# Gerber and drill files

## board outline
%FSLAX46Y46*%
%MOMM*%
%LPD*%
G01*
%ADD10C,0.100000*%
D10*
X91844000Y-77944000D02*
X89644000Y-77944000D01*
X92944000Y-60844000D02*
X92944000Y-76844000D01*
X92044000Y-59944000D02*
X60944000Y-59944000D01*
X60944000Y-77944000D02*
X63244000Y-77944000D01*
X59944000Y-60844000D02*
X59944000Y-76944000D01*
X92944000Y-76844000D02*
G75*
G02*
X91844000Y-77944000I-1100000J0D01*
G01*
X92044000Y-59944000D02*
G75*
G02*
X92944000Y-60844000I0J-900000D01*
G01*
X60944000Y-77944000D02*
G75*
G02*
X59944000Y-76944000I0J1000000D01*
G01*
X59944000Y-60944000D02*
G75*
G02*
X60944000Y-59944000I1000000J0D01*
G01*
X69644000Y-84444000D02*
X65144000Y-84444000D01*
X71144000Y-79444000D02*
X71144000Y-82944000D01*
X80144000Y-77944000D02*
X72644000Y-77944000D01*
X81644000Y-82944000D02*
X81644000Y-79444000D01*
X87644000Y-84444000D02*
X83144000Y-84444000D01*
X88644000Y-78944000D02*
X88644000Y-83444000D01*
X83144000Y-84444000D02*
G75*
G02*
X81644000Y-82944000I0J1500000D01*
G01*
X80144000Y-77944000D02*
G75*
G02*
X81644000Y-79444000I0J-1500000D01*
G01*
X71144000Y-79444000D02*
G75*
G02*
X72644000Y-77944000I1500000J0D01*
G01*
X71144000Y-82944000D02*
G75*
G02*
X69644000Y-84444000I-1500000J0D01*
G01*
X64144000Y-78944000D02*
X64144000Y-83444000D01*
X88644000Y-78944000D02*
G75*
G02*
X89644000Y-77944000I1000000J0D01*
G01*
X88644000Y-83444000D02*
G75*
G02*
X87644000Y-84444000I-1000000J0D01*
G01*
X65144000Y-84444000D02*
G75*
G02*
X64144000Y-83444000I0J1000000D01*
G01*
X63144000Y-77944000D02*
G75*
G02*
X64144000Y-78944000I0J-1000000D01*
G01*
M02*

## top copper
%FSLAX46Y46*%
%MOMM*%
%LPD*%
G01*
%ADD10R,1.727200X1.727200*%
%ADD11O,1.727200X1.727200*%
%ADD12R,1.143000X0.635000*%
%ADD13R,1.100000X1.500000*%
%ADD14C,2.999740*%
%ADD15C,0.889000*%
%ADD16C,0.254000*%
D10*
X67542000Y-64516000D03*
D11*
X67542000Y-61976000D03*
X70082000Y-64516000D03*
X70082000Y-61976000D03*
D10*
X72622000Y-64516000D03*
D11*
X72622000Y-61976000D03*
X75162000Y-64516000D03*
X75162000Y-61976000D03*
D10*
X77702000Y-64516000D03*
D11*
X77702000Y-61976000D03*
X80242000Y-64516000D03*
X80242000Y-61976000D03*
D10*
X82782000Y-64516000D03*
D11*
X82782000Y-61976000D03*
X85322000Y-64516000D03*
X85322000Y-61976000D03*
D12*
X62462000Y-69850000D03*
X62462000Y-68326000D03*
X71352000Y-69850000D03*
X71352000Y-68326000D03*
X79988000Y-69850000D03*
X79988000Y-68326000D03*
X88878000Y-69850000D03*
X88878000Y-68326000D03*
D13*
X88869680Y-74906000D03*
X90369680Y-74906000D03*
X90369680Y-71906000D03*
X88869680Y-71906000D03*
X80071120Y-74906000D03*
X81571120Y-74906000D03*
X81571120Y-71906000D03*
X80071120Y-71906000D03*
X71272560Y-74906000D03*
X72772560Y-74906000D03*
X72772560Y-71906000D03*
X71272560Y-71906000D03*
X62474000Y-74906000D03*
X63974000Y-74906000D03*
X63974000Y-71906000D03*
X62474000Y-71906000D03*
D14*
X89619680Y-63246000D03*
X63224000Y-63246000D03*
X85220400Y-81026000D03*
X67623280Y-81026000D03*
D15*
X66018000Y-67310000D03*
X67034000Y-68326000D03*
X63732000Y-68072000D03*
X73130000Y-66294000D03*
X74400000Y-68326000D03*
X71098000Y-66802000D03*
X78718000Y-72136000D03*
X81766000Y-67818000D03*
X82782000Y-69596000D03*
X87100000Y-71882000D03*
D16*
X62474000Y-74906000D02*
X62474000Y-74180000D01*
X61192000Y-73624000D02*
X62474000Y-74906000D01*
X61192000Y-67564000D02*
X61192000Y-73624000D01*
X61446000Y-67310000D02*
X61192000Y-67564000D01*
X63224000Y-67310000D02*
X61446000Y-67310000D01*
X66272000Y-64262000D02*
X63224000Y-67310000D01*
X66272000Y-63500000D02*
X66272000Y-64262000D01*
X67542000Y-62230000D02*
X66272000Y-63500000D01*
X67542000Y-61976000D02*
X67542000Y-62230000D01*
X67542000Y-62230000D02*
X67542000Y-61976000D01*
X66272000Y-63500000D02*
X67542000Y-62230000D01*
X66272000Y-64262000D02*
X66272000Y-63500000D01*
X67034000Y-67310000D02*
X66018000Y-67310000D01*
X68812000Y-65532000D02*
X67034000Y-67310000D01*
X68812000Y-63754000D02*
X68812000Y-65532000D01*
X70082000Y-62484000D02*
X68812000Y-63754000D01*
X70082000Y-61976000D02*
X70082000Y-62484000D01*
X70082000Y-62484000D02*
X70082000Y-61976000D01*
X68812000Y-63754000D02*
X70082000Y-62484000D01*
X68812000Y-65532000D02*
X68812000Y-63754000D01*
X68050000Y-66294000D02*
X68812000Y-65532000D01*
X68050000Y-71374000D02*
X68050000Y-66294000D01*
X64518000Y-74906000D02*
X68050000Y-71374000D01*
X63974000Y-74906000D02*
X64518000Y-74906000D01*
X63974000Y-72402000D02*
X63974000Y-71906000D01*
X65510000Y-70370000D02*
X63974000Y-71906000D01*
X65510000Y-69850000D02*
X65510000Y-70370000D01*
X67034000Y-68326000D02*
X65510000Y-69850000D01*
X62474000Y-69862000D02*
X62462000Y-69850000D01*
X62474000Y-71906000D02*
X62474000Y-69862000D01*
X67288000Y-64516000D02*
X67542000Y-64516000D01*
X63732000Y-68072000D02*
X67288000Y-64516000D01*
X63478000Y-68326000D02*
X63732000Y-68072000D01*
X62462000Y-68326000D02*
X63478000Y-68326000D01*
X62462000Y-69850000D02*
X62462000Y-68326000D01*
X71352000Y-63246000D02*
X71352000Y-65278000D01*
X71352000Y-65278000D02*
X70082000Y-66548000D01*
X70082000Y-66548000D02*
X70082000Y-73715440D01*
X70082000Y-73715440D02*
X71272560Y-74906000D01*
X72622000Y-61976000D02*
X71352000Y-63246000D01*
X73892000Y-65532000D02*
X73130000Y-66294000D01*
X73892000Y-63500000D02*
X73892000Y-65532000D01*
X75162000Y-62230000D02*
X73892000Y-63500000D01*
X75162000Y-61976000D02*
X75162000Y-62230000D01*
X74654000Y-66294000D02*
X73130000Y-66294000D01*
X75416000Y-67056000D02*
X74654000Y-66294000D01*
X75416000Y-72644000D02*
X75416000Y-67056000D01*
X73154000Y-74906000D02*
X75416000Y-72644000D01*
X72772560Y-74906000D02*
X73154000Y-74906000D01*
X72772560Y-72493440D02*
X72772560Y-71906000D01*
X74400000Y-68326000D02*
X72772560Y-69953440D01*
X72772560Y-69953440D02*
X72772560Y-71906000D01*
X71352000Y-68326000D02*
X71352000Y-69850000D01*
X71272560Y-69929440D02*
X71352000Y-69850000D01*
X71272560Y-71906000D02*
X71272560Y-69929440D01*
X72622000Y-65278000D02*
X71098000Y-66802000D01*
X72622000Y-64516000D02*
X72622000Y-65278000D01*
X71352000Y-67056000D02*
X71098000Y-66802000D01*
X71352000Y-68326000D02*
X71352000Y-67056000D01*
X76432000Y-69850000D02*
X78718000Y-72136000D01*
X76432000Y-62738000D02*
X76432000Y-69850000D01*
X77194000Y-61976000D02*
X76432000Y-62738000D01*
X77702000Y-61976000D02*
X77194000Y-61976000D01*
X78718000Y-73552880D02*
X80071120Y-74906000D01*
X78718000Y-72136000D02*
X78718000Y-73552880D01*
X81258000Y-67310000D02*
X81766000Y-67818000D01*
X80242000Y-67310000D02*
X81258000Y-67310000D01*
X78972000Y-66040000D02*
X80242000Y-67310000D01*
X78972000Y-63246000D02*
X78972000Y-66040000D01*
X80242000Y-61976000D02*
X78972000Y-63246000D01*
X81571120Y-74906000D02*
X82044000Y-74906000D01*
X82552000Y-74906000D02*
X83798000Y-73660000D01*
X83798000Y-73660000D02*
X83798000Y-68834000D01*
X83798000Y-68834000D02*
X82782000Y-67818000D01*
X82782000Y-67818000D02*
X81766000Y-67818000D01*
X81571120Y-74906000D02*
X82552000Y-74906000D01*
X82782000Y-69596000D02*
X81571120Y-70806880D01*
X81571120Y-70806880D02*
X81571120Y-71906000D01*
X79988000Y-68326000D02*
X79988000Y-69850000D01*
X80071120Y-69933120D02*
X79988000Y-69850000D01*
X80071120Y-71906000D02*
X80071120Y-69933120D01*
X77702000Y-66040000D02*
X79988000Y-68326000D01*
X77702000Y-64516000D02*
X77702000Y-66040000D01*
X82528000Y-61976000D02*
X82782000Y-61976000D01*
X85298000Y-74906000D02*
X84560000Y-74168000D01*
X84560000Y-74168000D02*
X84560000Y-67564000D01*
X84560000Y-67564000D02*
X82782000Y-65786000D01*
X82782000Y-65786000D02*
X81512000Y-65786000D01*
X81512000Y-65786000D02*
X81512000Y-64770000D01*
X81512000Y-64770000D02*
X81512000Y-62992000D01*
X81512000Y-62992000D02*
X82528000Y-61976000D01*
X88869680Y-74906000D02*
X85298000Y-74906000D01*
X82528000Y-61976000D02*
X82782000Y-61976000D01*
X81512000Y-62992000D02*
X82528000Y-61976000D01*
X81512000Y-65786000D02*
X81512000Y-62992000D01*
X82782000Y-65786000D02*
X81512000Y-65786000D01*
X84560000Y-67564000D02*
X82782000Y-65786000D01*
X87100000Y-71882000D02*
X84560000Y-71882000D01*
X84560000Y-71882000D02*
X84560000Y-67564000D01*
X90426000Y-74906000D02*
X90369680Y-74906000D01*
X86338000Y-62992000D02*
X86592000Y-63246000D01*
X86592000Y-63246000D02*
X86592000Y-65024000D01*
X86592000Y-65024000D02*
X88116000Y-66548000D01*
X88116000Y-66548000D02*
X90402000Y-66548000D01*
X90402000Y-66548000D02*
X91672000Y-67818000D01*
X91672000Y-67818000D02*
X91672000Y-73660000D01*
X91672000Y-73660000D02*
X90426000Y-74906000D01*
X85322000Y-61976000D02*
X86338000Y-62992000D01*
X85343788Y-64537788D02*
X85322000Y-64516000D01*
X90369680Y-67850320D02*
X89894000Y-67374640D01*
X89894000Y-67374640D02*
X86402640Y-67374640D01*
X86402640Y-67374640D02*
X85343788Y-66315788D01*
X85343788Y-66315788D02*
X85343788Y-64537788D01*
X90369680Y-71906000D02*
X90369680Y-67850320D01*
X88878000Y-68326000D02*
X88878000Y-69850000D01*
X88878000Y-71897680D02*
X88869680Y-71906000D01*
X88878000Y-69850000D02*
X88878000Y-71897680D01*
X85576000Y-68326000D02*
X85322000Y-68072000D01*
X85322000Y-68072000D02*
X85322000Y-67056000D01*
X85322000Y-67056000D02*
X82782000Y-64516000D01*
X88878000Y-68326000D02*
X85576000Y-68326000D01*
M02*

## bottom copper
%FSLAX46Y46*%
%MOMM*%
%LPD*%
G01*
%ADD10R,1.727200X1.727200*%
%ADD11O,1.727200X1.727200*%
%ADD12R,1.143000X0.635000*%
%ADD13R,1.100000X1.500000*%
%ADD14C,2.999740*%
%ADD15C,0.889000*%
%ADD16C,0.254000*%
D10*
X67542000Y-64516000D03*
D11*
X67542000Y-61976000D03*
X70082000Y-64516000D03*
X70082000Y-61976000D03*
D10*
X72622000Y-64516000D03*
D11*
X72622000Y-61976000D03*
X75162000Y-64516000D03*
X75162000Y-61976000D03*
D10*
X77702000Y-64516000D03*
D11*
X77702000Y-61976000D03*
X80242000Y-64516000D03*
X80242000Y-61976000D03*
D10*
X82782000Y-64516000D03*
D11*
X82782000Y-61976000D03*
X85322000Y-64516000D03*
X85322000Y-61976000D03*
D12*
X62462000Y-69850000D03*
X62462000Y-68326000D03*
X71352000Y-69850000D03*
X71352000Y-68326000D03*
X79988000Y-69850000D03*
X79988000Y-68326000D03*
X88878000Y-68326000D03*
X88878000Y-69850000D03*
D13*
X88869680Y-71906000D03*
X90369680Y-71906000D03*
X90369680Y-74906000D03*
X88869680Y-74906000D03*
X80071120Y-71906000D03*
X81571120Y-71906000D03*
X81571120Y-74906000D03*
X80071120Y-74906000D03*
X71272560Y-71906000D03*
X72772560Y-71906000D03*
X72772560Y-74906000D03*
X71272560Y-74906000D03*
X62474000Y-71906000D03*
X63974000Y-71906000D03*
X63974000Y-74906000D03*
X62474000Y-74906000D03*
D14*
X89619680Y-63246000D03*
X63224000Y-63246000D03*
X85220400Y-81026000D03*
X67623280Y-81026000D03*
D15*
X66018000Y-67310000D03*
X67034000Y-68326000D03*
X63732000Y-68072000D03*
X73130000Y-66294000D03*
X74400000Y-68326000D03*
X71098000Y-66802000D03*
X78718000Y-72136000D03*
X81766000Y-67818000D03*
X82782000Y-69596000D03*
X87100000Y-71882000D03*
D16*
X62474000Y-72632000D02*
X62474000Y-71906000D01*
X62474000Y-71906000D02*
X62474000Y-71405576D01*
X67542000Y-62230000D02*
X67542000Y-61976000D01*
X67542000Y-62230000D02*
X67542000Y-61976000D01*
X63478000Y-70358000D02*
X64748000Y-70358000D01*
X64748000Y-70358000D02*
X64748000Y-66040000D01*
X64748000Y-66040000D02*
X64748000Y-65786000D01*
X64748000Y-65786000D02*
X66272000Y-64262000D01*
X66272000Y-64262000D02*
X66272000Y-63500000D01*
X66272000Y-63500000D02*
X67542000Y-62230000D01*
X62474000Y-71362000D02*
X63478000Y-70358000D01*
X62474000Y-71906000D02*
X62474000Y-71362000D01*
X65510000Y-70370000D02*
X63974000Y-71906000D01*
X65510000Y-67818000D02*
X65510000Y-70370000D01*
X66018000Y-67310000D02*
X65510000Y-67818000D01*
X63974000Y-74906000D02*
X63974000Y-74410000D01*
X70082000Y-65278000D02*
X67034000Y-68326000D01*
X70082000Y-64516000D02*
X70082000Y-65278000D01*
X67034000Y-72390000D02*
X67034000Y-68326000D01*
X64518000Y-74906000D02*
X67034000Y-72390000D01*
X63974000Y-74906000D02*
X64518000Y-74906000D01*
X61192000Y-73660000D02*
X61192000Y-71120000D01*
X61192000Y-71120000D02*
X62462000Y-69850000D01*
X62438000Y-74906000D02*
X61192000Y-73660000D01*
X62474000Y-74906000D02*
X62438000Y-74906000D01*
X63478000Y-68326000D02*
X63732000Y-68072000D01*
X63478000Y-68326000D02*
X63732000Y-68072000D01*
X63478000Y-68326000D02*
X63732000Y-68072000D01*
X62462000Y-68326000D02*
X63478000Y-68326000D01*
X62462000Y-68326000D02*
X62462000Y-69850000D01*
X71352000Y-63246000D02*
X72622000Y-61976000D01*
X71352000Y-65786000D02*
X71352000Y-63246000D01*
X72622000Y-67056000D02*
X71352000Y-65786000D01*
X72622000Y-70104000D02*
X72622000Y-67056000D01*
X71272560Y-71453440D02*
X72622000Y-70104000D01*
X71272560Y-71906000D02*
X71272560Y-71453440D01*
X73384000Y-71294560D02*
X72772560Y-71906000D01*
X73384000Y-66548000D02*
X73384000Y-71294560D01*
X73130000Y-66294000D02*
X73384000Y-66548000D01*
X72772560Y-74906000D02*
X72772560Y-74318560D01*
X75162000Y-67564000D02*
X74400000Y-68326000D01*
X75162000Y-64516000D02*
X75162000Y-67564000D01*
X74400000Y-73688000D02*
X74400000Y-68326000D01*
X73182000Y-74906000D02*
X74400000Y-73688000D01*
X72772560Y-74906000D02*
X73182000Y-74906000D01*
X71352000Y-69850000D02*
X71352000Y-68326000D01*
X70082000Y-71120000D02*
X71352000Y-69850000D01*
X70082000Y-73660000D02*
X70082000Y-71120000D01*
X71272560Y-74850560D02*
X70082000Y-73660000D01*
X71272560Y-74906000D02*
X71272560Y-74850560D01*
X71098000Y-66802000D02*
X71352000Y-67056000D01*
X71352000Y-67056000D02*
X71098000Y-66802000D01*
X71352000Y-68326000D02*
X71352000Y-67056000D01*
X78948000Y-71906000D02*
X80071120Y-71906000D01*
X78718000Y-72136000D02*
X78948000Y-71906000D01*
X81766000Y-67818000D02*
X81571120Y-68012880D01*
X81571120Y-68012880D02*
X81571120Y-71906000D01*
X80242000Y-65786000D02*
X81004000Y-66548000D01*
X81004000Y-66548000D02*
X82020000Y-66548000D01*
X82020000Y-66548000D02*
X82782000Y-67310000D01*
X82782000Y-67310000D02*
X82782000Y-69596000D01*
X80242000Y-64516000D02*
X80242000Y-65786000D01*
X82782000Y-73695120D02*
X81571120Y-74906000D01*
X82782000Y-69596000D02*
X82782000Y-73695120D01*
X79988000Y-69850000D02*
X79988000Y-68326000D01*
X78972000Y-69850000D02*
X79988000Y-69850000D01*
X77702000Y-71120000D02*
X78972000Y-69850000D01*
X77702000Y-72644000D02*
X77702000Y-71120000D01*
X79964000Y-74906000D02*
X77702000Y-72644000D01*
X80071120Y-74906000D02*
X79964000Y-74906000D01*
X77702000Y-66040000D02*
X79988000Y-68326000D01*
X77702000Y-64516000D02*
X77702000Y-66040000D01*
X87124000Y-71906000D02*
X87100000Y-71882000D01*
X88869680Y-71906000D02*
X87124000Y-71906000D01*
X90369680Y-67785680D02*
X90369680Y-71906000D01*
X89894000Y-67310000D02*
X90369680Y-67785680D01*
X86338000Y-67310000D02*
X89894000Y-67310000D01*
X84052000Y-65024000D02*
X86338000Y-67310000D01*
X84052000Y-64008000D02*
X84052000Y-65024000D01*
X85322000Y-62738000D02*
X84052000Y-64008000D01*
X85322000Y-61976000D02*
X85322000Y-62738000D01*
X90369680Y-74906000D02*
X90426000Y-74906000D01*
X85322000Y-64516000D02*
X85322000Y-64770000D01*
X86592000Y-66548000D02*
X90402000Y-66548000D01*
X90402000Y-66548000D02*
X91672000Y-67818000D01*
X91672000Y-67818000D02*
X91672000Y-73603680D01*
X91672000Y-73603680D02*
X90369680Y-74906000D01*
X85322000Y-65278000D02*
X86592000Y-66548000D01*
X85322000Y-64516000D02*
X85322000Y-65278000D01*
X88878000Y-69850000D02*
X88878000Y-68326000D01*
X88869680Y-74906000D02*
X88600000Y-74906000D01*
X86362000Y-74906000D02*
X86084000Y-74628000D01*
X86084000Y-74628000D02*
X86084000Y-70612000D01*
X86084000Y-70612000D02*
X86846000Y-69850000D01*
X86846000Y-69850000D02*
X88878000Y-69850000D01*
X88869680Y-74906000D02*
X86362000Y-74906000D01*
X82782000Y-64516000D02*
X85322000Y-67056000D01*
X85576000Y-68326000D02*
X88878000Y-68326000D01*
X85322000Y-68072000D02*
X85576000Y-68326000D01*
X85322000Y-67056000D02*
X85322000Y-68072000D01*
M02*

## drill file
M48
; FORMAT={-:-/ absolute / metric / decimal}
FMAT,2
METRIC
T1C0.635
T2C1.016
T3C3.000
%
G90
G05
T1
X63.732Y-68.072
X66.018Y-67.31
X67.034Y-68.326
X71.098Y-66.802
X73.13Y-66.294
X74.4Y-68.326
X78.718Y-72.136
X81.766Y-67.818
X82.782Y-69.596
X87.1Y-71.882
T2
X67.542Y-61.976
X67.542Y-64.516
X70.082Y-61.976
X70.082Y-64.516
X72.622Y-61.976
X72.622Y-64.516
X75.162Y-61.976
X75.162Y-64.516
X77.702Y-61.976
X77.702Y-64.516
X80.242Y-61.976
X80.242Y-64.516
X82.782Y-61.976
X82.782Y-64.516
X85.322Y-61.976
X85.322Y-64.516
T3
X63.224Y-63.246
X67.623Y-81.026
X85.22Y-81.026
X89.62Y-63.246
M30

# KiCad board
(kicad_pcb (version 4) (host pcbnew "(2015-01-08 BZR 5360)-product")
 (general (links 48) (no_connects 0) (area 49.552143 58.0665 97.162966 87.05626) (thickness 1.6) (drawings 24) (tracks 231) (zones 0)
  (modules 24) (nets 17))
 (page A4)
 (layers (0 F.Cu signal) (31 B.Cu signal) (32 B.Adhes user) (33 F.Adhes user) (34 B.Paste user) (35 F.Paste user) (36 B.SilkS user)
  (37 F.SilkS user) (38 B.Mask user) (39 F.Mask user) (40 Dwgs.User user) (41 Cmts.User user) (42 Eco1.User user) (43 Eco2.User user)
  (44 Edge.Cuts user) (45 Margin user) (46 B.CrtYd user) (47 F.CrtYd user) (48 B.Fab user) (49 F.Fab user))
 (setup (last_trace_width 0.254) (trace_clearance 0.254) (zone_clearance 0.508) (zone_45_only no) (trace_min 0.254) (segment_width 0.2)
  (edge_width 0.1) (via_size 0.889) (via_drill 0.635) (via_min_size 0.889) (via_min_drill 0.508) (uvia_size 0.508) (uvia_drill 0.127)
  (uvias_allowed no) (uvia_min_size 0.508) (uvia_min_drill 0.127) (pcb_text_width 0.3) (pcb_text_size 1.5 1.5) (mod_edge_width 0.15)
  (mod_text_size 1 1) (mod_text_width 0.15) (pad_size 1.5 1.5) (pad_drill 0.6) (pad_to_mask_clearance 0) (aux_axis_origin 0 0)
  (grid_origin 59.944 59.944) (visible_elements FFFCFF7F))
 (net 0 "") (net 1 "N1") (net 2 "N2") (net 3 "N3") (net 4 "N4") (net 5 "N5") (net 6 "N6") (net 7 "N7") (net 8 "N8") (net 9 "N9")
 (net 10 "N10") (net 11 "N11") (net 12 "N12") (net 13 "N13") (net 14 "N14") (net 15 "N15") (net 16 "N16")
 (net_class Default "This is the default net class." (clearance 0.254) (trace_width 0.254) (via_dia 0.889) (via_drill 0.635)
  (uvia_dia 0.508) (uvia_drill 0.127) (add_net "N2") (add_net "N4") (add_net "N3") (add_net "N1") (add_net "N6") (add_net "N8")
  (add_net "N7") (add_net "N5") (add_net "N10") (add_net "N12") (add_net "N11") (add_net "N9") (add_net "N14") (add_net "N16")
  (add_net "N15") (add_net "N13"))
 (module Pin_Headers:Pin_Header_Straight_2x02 (layer F.Cu) (at 68.812 63.246)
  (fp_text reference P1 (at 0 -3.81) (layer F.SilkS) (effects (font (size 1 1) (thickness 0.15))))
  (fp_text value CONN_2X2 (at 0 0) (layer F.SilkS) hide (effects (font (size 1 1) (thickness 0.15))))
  (pad 1 thru_hole rect (at -1.27 1.27) (size 1.7272 1.7272) (drill 1.016) (layers *.Cu *.Mask F.SilkS) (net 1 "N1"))
  (pad 2 thru_hole oval (at -1.27 -1.27) (size 1.7272 1.7272) (drill 1.016) (layers *.Cu *.Mask F.SilkS) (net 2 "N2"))
  (pad 3 thru_hole oval (at 1.27 1.27) (size 1.7272 1.7272) (drill 1.016) (layers *.Cu *.Mask F.SilkS) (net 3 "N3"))
  (pad 4 thru_hole oval (at 1.27 -1.27) (size 1.7272 1.7272) (drill 1.016) (layers *.Cu *.Mask F.SilkS) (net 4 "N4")))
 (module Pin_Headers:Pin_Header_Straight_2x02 (layer F.Cu) (at 73.892 63.246)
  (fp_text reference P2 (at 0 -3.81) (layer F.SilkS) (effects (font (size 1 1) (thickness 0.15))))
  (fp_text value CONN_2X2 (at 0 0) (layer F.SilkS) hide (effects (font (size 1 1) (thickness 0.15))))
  (pad 1 thru_hole rect (at -1.27 1.27) (size 1.7272 1.7272) (drill 1.016) (layers *.Cu *.Mask F.SilkS) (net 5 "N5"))
  (pad 2 thru_hole oval (at -1.27 -1.27) (size 1.7272 1.7272) (drill 1.016) (layers *.Cu *.Mask F.SilkS) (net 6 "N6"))
  (pad 3 thru_hole oval (at 1.27 1.27) (size 1.7272 1.7272) (drill 1.016) (layers *.Cu *.Mask F.SilkS) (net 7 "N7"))
  (pad 4 thru_hole oval (at 1.27 -1.27) (size 1.7272 1.7272) (drill 1.016) (layers *.Cu *.Mask F.SilkS) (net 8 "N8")))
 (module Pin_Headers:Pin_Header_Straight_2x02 (layer F.Cu) (at 78.972 63.246)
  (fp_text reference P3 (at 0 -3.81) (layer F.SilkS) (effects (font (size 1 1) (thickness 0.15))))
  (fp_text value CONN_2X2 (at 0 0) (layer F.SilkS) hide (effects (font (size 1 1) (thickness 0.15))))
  (pad 1 thru_hole rect (at -1.27 1.27) (size 1.7272 1.7272) (drill 1.016) (layers *.Cu *.Mask F.SilkS) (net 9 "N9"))
  (pad 2 thru_hole oval (at -1.27 -1.27) (size 1.7272 1.7272) (drill 1.016) (layers *.Cu *.Mask F.SilkS) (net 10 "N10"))
  (pad 3 thru_hole oval (at 1.27 1.27) (size 1.7272 1.7272) (drill 1.016) (layers *.Cu *.Mask F.SilkS) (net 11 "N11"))
  (pad 4 thru_hole oval (at 1.27 -1.27) (size 1.7272 1.7272) (drill 1.016) (layers *.Cu *.Mask F.SilkS) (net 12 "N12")))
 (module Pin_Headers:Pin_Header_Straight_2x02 (layer F.Cu) (at 84.052 63.246)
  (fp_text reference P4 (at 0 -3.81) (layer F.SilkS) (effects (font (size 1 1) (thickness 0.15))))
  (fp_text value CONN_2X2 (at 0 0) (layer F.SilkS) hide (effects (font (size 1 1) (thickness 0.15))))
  (pad 1 thru_hole rect (at -1.27 1.27) (size 1.7272 1.7272) (drill 1.016) (layers *.Cu *.Mask F.SilkS) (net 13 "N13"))
  (pad 2 thru_hole oval (at -1.27 -1.27) (size 1.7272 1.7272) (drill 1.016) (layers *.Cu *.Mask F.SilkS) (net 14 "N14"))
  (pad 3 thru_hole oval (at 1.27 1.27) (size 1.7272 1.7272) (drill 1.016) (layers *.Cu *.Mask F.SilkS) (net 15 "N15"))
  (pad 4 thru_hole oval (at 1.27 -1.27) (size 1.7272 1.7272) (drill 1.016) (layers *.Cu *.Mask F.SilkS) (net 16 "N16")))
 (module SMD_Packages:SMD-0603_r (layer F.Cu) (at 62.462 69.088 90)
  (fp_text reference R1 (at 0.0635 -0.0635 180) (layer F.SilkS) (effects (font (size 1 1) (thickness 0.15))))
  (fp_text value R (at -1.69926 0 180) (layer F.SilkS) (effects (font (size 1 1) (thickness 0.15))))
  (pad 1 smd rect (at -0.762 0 90) (size 0.635 1.143) (layers F.Cu F.Paste F.Mask) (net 1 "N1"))
  (pad 2 smd rect (at 0.762 0 90) (size 0.635 1.143) (layers F.Cu F.Paste F.Mask) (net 1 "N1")))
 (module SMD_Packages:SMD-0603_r (layer B.Cu) (at 62.462 69.088 90)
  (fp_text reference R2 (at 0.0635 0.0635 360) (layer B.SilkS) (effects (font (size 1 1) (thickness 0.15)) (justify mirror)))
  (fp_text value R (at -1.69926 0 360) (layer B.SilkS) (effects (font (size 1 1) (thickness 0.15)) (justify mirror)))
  (pad 1 smd rect (at -0.762 0 90) (size 0.635 1.143) (layers B.Cu B.Paste B.Mask) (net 1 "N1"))
  (pad 2 smd rect (at 0.762 0 90) (size 0.635 1.143) (layers B.Cu B.Paste B.Mask) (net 1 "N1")))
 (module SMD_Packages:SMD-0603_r (layer F.Cu) (at 71.352 69.088 90)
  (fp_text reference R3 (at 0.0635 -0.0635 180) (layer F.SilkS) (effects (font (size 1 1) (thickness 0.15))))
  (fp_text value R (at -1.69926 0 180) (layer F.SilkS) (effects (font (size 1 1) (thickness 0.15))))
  (pad 1 smd rect (at -0.762 0 90) (size 0.635 1.143) (layers F.Cu F.Paste F.Mask) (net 5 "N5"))
  (pad 2 smd rect (at 0.762 0 90) (size 0.635 1.143) (layers F.Cu F.Paste F.Mask) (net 5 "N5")))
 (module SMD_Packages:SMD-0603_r (layer B.Cu) (at 71.352 69.088 90)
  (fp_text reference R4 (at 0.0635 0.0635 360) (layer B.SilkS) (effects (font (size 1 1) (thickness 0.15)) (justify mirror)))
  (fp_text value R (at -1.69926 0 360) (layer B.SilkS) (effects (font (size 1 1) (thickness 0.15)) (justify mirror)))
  (pad 1 smd rect (at -0.762 0 90) (size 0.635 1.143) (layers B.Cu B.Paste B.Mask) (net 5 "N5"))
  (pad 2 smd rect (at 0.762 0 90) (size 0.635 1.143) (layers B.Cu B.Paste B.Mask) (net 5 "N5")))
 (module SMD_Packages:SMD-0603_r (layer F.Cu) (at 79.988 69.088 90)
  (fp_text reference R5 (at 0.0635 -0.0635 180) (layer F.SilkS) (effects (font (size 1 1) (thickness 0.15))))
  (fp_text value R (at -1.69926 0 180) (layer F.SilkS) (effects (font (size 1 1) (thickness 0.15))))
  (pad 1 smd rect (at -0.762 0 90) (size 0.635 1.143) (layers F.Cu F.Paste F.Mask) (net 9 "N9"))
  (pad 2 smd rect (at 0.762 0 90) (size 0.635 1.143) (layers F.Cu F.Paste F.Mask) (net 9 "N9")))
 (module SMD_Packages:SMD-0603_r (layer B.Cu) (at 79.988 69.088 90)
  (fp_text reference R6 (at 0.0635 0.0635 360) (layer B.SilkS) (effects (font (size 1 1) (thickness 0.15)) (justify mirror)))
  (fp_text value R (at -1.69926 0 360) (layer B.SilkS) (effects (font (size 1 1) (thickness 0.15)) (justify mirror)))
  (pad 1 smd rect (at -0.762 0 90) (size 0.635 1.143) (layers B.Cu B.Paste B.Mask) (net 9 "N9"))
  (pad 2 smd rect (at 0.762 0 90) (size 0.635 1.143) (layers B.Cu B.Paste B.Mask) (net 9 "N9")))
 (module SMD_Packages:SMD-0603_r (layer F.Cu) (at 88.878 69.088 90)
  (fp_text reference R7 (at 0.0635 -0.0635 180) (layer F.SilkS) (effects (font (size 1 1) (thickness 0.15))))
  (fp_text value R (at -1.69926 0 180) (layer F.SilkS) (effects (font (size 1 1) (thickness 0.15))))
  (pad 1 smd rect (at -0.762 0 90) (size 0.635 1.143) (layers F.Cu F.Paste F.Mask) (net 13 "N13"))
  (pad 2 smd rect (at 0.762 0 90) (size 0.635 1.143) (layers F.Cu F.Paste F.Mask) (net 13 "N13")))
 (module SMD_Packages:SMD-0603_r (layer B.Cu) (at 88.878 69.088 270)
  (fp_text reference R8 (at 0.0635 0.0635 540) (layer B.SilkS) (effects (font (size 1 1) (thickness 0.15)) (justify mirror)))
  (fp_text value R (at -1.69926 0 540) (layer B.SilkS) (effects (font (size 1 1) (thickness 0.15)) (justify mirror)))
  (pad 1 smd rect (at -0.762 0 270) (size 0.635 1.143) (layers B.Cu B.Paste B.Mask) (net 13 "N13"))
  (pad 2 smd rect (at 0.762 0 270) (size 0.635 1.143) (layers B.Cu B.Paste B.Mask) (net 13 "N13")))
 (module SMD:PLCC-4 (layer B.Cu) (at 89.61968 73.406 270)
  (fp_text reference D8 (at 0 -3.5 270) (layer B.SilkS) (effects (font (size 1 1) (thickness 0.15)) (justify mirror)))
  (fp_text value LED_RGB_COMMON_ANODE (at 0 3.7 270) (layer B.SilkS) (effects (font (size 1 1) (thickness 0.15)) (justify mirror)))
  (pad 1 smd rect (at -1.5 0.75) (size 1.1 1.5) (layers B.Cu B.Paste B.Mask) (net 14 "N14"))
  (pad 2 smd rect (at -1.5 -0.75) (size 1.1 1.5) (layers B.Cu B.Paste B.Mask) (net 16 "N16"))
  (pad 3 smd rect (at 1.5 -0.75) (size 1.1 1.5) (layers B.Cu B.Paste B.Mask) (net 15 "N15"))
  (pad 4 smd rect (at 1.5 0.75) (size 1.1 1.5) (layers B.Cu B.Paste B.Mask) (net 13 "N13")))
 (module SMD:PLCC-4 (layer F.Cu) (at 89.61968 73.406 90)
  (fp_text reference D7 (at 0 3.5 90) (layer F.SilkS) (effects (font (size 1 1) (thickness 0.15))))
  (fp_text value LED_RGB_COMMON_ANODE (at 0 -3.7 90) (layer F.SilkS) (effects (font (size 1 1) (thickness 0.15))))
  (pad 1 smd rect (at -1.5 -0.75) (size 1.1 1.5) (layers F.Cu F.Paste F.Mask) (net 14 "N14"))
  (pad 2 smd rect (at -1.5 0.75) (size 1.1 1.5) (layers F.Cu F.Paste F.Mask) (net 16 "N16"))
  (pad 3 smd rect (at 1.5 0.75) (size 1.1 1.5) (layers F.Cu F.Paste F.Mask) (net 15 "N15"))
  (pad 4 smd rect (at 1.5 -0.75) (size 1.1 1.5) (layers F.Cu F.Paste F.Mask) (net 13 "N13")))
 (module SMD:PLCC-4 (layer B.Cu) (at 80.82112 73.406 270)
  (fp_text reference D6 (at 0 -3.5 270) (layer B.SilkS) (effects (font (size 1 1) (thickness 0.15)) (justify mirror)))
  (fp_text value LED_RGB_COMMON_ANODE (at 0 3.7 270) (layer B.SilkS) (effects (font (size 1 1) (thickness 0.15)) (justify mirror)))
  (pad 1 smd rect (at -1.5 0.75) (size 1.1 1.5) (layers B.Cu B.Paste B.Mask) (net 10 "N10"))
  (pad 2 smd rect (at -1.5 -0.75) (size 1.1 1.5) (layers B.Cu B.Paste B.Mask) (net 12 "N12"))
  (pad 3 smd rect (at 1.5 -0.75) (size 1.1 1.5) (layers B.Cu B.Paste B.Mask) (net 11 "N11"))
  (pad 4 smd rect (at 1.5 0.75) (size 1.1 1.5) (layers B.Cu B.Paste B.Mask) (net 9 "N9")))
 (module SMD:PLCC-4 (layer F.Cu) (at 80.82112 73.406 90)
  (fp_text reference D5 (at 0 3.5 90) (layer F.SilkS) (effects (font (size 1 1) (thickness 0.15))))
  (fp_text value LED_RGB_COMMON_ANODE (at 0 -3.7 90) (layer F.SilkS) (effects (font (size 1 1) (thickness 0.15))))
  (pad 1 smd rect (at -1.5 -0.75) (size 1.1 1.5) (layers F.Cu F.Paste F.Mask) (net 10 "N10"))
  (pad 2 smd rect (at -1.5 0.75) (size 1.1 1.5) (layers F.Cu F.Paste F.Mask) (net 12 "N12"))
  (pad 3 smd rect (at 1.5 0.75) (size 1.1 1.5) (layers F.Cu F.Paste F.Mask) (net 11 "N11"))
  (pad 4 smd rect (at 1.5 -0.75) (size 1.1 1.5) (layers F.Cu F.Paste F.Mask) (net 9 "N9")))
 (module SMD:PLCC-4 (layer B.Cu) (at 72.02256 73.406 270)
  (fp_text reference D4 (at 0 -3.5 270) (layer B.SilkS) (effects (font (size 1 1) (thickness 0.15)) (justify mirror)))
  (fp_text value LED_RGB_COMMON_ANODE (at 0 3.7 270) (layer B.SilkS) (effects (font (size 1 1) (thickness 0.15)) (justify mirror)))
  (pad 1 smd rect (at -1.5 0.75) (size 1.1 1.5) (layers B.Cu B.Paste B.Mask) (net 6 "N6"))
  (pad 2 smd rect (at -1.5 -0.75) (size 1.1 1.5) (layers B.Cu B.Paste B.Mask) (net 8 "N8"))
  (pad 3 smd rect (at 1.5 -0.75) (size 1.1 1.5) (layers B.Cu B.Paste B.Mask) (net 7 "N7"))
  (pad 4 smd rect (at 1.5 0.75) (size 1.1 1.5) (layers B.Cu B.Paste B.Mask) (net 5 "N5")))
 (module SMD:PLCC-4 (layer F.Cu) (at 72.02256 73.406 90)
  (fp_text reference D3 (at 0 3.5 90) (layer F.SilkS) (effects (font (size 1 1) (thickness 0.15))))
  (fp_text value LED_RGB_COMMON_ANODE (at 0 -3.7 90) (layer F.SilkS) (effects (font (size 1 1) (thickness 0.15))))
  (pad 1 smd rect (at -1.5 -0.75) (size 1.1 1.5) (layers F.Cu F.Paste F.Mask) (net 6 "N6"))
  (pad 2 smd rect (at -1.5 0.75) (size 1.1 1.5) (layers F.Cu F.Paste F.Mask) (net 8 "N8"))
  (pad 3 smd rect (at 1.5 0.75) (size 1.1 1.5) (layers F.Cu F.Paste F.Mask) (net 7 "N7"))
  (pad 4 smd rect (at 1.5 -0.75) (size 1.1 1.5) (layers F.Cu F.Paste F.Mask) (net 5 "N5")))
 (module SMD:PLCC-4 (layer B.Cu) (at 63.224 73.406 270)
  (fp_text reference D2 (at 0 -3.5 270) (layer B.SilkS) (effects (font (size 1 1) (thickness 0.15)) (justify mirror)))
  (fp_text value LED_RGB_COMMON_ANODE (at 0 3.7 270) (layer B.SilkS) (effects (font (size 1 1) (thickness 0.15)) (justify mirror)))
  (pad 1 smd rect (at -1.5 0.75) (size 1.1 1.5) (layers B.Cu B.Paste B.Mask) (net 2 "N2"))
  (pad 2 smd rect (at -1.5 -0.75) (size 1.1 1.5) (layers B.Cu B.Paste B.Mask) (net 4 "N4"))
  (pad 3 smd rect (at 1.5 -0.75) (size 1.1 1.5) (layers B.Cu B.Paste B.Mask) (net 3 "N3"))
  (pad 4 smd rect (at 1.5 0.75) (size 1.1 1.5) (layers B.Cu B.Paste B.Mask) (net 1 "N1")))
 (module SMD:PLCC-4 (layer F.Cu) (at 63.224 73.406 90)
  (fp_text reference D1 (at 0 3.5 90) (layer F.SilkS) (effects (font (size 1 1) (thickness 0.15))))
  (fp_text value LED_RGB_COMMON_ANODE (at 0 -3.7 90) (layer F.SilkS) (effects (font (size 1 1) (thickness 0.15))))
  (pad 1 smd rect (at -1.5 -0.75) (size 1.1 1.5) (layers F.Cu F.Paste F.Mask) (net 2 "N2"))
  (pad 2 smd rect (at -1.5 0.75) (size 1.1 1.5) (layers F.Cu F.Paste F.Mask) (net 4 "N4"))
  (pad 3 smd rect (at 1.5 0.75) (size 1.1 1.5) (layers F.Cu F.Paste F.Mask) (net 3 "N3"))
  (pad 4 smd rect (at 1.5 -0.75) (size 1.1 1.5) (layers F.Cu F.Paste F.Mask) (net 1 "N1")))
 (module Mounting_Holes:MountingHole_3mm (layer F.Cu) (at 89.61968 63.246)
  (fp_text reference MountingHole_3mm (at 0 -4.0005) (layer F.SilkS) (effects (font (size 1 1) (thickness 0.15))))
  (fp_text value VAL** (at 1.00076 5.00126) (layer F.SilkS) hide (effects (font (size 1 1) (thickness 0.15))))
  (pad 1 thru_hole circle (at 0 0) (size 2.99974 2.99974) (drill 2.99974) (layers)))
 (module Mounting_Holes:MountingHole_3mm (layer F.Cu) (at 63.224 63.246)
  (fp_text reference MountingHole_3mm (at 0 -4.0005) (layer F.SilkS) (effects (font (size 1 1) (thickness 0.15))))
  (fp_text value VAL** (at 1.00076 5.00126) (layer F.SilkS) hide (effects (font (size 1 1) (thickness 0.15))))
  (pad 1 thru_hole circle (at 0 0) (size 2.99974 2.99974) (drill 2.99974) (layers)))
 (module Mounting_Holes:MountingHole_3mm (layer F.Cu) (at 85.2204 81.026)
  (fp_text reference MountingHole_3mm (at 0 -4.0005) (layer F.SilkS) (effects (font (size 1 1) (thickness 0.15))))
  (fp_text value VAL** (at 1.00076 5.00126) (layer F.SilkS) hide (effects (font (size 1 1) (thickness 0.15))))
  (pad 1 thru_hole circle (at 0 0) (size 2.99974 2.99974) (drill 2.99974) (layers)))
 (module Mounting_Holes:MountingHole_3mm (layer F.Cu) (at 67.62328 81.026)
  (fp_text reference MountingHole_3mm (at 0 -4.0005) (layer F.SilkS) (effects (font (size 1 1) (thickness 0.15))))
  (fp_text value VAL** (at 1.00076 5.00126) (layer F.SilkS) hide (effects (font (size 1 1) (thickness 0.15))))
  (pad 1 thru_hole circle (at 0 0) (size 2.99974 2.99974) (drill 2.99974) (layers)))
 (gr_line (start 91.844 77.944) (end 89.644 77.944) (angle 90) (layer Edge.Cuts) (width 0.1))
 (gr_line (start 92.944 60.844) (end 92.944 76.844) (angle 90) (layer Edge.Cuts) (width 0.1))
 (gr_line (start 92.044 59.944) (end 60.944 59.944) (angle 90) (layer Edge.Cuts) (width 0.1))
 (gr_line (start 60.944 77.944) (end 63.244 77.944) (angle 90) (layer Edge.Cuts) (width 0.1))
 (gr_line (start 59.944 60.844) (end 59.944 76.944) (angle 90) (layer Edge.Cuts) (width 0.1))
 (gr_arc (start 91.844 76.844) (end 92.944 76.844) (angle 90) (layer Edge.Cuts) (width 0.1))
 (gr_arc (start 92.044 60.844) (end 92.044 59.944) (angle 90) (layer Edge.Cuts) (width 0.1))
 (gr_arc (start 60.944 76.944) (end 60.944 77.944) (angle 90) (layer Edge.Cuts) (width 0.1))
 (gr_arc (start 60.944 60.944) (end 59.944 60.944) (angle 90) (layer Edge.Cuts) (width 0.1))
 (gr_line (start 69.644 84.444) (end 65.144 84.444) (angle 90) (layer Edge.Cuts) (width 0.1))
 (gr_line (start 71.144 79.444) (end 71.144 82.944) (angle 90) (layer Edge.Cuts) (width 0.1))
 (gr_line (start 80.144 77.944) (end 72.644 77.944) (angle 90) (layer Edge.Cuts) (width 0.1))
 (gr_line (start 81.644 82.944) (end 81.644 79.444) (angle 90) (layer Edge.Cuts) (width 0.1))
 (gr_line (start 87.644 84.444) (end 83.144 84.444) (angle 90) (layer Edge.Cuts) (width 0.1))
 (gr_line (start 88.644 78.944) (end 88.644 83.444) (angle 90) (layer Edge.Cuts) (width 0.1))
 (gr_arc (start 83.144 82.944) (end 83.144 84.444) (angle 90) (layer Edge.Cuts) (width 0.1))
 (gr_arc (start 80.144 79.444) (end 80.144 77.944) (angle 90) (layer Edge.Cuts) (width 0.1))
 (gr_arc (start 72.644 79.444) (end 71.144 79.444) (angle 90) (layer Edge.Cuts) (width 0.1))
 (gr_arc (start 69.644 82.944) (end 71.144 82.944) (angle 90) (layer Edge.Cuts) (width 0.1))
 (gr_line (start 64.144 78.944) (end 64.144 83.444) (angle 90) (layer Edge.Cuts) (width 0.1))
 (gr_arc (start 89.644 78.944) (end 88.644 78.944) (angle 90) (layer Edge.Cuts) (width 0.1))
 (gr_arc (start 87.644 83.444) (end 88.644 83.444) (angle 90) (layer Edge.Cuts) (width 0.1))
 (gr_arc (start 65.144 83.444) (end 65.144 84.444) (angle 90) (layer Edge.Cuts) (width 0.1))
 (gr_arc (start 63.144 78.944) (end 63.144 77.944) (angle 90) (layer Edge.Cuts) (width 0.1))
 (segment (start 62.474 72.632) (end 62.474 71.906) (width 0.254) (layer B.Cu) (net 2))
 (segment (start 62.474 74.906) (end 62.474 74.18) (width 0.254) (layer F.Cu) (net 2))
 (segment (start 62.474 71.906) (end 62.474 71.405576) (width 0.254) (layer B.Cu) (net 2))
 (segment (start 61.192 73.624) (end 62.474 74.906) (width 0.254) (layer F.Cu) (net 2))
 (segment (start 61.192 67.564) (end 61.192 73.624) (width 0.254) (layer F.Cu) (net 2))
 (segment (start 61.446 67.31) (end 61.192 67.564) (width 0.254) (layer F.Cu) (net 2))
 (segment (start 63.224 67.31) (end 61.446 67.31) (width 0.254) (layer F.Cu) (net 2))
 (segment (start 66.272 64.262) (end 63.224 67.31) (width 0.254) (layer F.Cu) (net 2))
 (segment (start 66.272 63.5) (end 66.272 64.262) (width 0.254) (layer F.Cu) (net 2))
 (segment (start 67.542 62.23) (end 66.272 63.5) (width 0.254) (layer F.Cu) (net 2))
 (segment (start 67.542 61.976) (end 67.542 62.23) (width 0.254) (layer F.Cu) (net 2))
 (segment (start 67.542 62.23) (end 67.542 61.976) (width 0.254) (layer F.Cu) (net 2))
 (segment (start 66.272 63.5) (end 67.542 62.23) (width 0.254) (layer F.Cu) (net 2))
 (segment (start 66.272 64.262) (end 66.272 63.5) (width 0.254) (layer F.Cu) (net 2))
 (segment (start 67.542 62.23) (end 67.542 61.976) (width 0.254) (layer B.Cu) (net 2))
 (segment (start 67.542 62.23) (end 67.542 61.976) (width 0.254) (layer B.Cu) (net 2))
 (segment (start 63.478 70.358) (end 64.748 70.358) (width 0.254) (layer B.Cu) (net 2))
 (segment (start 64.748 70.358) (end 64.748 66.04) (width 0.254) (layer B.Cu) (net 2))
 (segment (start 64.748 66.04) (end 64.748 65.786) (width 0.254) (layer B.Cu) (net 2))
 (segment (start 64.748 65.786) (end 66.272 64.262) (width 0.254) (layer B.Cu) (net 2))
 (segment (start 66.272 64.262) (end 66.272 63.5) (width 0.254) (layer B.Cu) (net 2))
 (segment (start 66.272 63.5) (end 67.542 62.23) (width 0.254) (layer B.Cu) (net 2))
 (segment (start 62.474 71.362) (end 63.478 70.358) (width 0.254) (layer B.Cu) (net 2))
 (segment (start 62.474 71.906) (end 62.474 71.362) (width 0.254) (layer B.Cu) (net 2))
 (segment (start 65.51 70.37) (end 63.974 71.906) (width 0.254) (layer B.Cu) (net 4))
 (segment (start 65.51 67.818) (end 65.51 70.37) (width 0.254) (layer B.Cu) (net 4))
 (segment (start 66.018 67.31) (end 65.51 67.818) (width 0.254) (layer B.Cu) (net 4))
 (via (at 66.018 67.31) (size 0.889) (layers F.Cu B.Cu) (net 4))
 (segment (start 67.034 67.31) (end 66.018 67.31) (width 0.254) (layer F.Cu) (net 4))
 (segment (start 68.812 65.532) (end 67.034 67.31) (width 0.254) (layer F.Cu) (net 4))
 (segment (start 68.812 63.754) (end 68.812 65.532) (width 0.254) (layer F.Cu) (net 4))
 (segment (start 70.082 62.484) (end 68.812 63.754) (width 0.254) (layer F.Cu) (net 4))
 (segment (start 70.082 61.976) (end 70.082 62.484) (width 0.254) (layer F.Cu) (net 4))
 (segment (start 70.082 62.484) (end 70.082 61.976) (width 0.254) (layer F.Cu) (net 4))
 (segment (start 68.812 63.754) (end 70.082 62.484) (width 0.254) (layer F.Cu) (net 4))
 (segment (start 68.812 65.532) (end 68.812 63.754) (width 0.254) (layer F.Cu) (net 4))
 (segment (start 68.05 66.294) (end 68.812 65.532) (width 0.254) (layer F.Cu) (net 4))
 (segment (start 68.05 71.374) (end 68.05 66.294) (width 0.254) (layer F.Cu) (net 4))
 (segment (start 64.518 74.906) (end 68.05 71.374) (width 0.254) (layer F.Cu) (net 4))
 (segment (start 63.974 74.906) (end 64.518 74.906) (width 0.254) (layer F.Cu) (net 4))
 (segment (start 63.974 72.402) (end 63.974 71.906) (width 0.254) (layer F.Cu) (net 3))
 (segment (start 63.974 74.906) (end 63.974 74.41) (width 0.254) (layer B.Cu) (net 3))
 (segment (start 65.51 70.37) (end 63.974 71.906) (width 0.254) (layer F.Cu) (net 3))
 (segment (start 65.51 69.85) (end 65.51 70.37) (width 0.254) (layer F.Cu) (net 3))
 (segment (start 67.034 68.326) (end 65.51 69.85) (width 0.254) (layer F.Cu) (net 3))
 (via (at 67.034 68.326) (size 0.889) (layers F.Cu B.Cu) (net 3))
 (segment (start 70.082 65.278) (end 67.034 68.326) (width 0.254) (layer B.Cu) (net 3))
 (segment (start 70.082 64.516) (end 70.082 65.278) (width 0.254) (layer B.Cu) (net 3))
 (segment (start 67.034 72.39) (end 67.034 68.326) (width 0.254) (layer B.Cu) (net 3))
 (segment (start 64.518 74.906) (end 67.034 72.39) (width 0.254) (layer B.Cu) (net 3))
 (segment (start 63.974 74.906) (end 64.518 74.906) (width 0.254) (layer B.Cu) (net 3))
 (segment (start 62.474 69.862) (end 62.462 69.85) (width 0.254) (layer F.Cu) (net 1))
 (segment (start 62.474 71.906) (end 62.474 69.862) (width 0.254) (layer F.Cu) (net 1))
 (segment (start 61.192 73.66) (end 61.192 71.12) (width 0.254) (layer B.Cu) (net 1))
 (segment (start 61.192 71.12) (end 62.462 69.85) (width 0.254) (layer B.Cu) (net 1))
 (segment (start 62.438 74.906) (end 61.192 73.66) (width 0.254) (layer B.Cu) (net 1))
 (segment (start 62.474 74.906) (end 62.438 74.906) (width 0.254) (layer B.Cu) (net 1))
 (segment (start 67.288 64.516) (end 67.542 64.516) (width 0.254) (layer F.Cu) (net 1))
 (segment (start 63.478 68.326) (end 63.732 68.072) (width 0.254) (layer B.Cu) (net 1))
 (via (at 63.732 68.072) (size 0.889) (layers F.Cu B.Cu) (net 1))
 (segment (start 63.732 68.072) (end 67.288 64.516) (width 0.254) (layer F.Cu) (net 1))
 (segment (start 63.478 68.326) (end 63.732 68.072) (width 0.254) (layer B.Cu) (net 1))
 (segment (start 63.478 68.326) (end 63.732 68.072) (width 0.254) (layer F.Cu) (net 1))
 (segment (start 62.462 68.326) (end 63.478 68.326) (width 0.254) (layer F.Cu) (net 1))
 (segment (start 63.478 68.326) (end 63.732 68.072) (width 0.254) (layer B.Cu) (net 1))
 (segment (start 62.462 68.326) (end 63.478 68.326) (width 0.254) (layer B.Cu) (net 1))
 (segment (start 62.462 68.326) (end 62.462 69.85) (width 0.254) (layer B.Cu) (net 1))
 (segment (start 62.462 69.85) (end 62.462 68.326) (width 0.254) (layer F.Cu) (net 1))
 (segment (start 71.352 63.246) (end 71.352 65.278) (width 0.254) (layer F.Cu) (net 6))
 (segment (start 71.352 65.278) (end 70.082 66.548) (width 0.254) (layer F.Cu) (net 6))
 (segment (start 70.082 66.548) (end 70.082 73.71544) (width 0.254) (layer F.Cu) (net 6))
 (segment (start 70.082 73.71544) (end 71.27256 74.906) (width 0.254) (layer F.Cu) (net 6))
 (segment (start 72.622 61.976) (end 71.352 63.246) (width 0.254) (layer F.Cu) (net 6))
 (segment (start 71.352 63.246) (end 72.622 61.976) (width 0.254) (layer B.Cu) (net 6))
 (segment (start 71.352 65.786) (end 71.352 63.246) (width 0.254) (layer B.Cu) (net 6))
 (segment (start 72.622 67.056) (end 71.352 65.786) (width 0.254) (layer B.Cu) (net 6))
 (segment (start 72.622 70.104) (end 72.622 67.056) (width 0.254) (layer B.Cu) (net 6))
 (segment (start 71.27256 71.45344) (end 72.622 70.104) (width 0.254) (layer B.Cu) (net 6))
 (segment (start 71.27256 71.906) (end 71.27256 71.45344) (width 0.254) (layer B.Cu) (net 6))
 (segment (start 73.384 71.29456) (end 72.77256 71.906) (width 0.254) (layer B.Cu) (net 8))
 (segment (start 73.384 66.548) (end 73.384 71.29456) (width 0.254) (layer B.Cu) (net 8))
 (segment (start 73.13 66.294) (end 73.384 66.548) (width 0.254) (layer B.Cu) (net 8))
 (via (at 73.13 66.294) (size 0.889) (layers F.Cu B.Cu) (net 8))
 (segment (start 73.892 65.532) (end 73.13 66.294) (width 0.254) (layer F.Cu) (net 8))
 (segment (start 73.892 63.5) (end 73.892 65.532) (width 0.254) (layer F.Cu) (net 8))
 (segment (start 75.162 62.23) (end 73.892 63.5) (width 0.254) (layer F.Cu) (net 8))
 (segment (start 75.162 61.976) (end 75.162 62.23) (width 0.254) (layer F.Cu) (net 8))
 (segment (start 74.654 66.294) (end 73.13 66.294) (width 0.254) (layer F.Cu) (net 8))
 (segment (start 75.416 67.056) (end 74.654 66.294) (width 0.254) (layer F.Cu) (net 8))
 (segment (start 75.416 72.644) (end 75.416 67.056) (width 0.254) (layer F.Cu) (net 8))
 (segment (start 73.154 74.906) (end 75.416 72.644) (width 0.254) (layer F.Cu) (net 8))
 (segment (start 72.77256 74.906) (end 73.154 74.906) (width 0.254) (layer F.Cu) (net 8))
 (segment (start 72.77256 72.49344) (end 72.77256 71.906) (width 0.254) (layer F.Cu) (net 7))
 (segment (start 72.77256 74.906) (end 72.77256 74.31856) (width 0.254) (layer B.Cu) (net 7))
 (segment (start 75.162 67.564) (end 74.4 68.326) (width 0.254) (layer B.Cu) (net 7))
 (via (at 74.4 68.326) (size 0.889) (layers F.Cu B.Cu) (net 7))
 (segment (start 74.4 68.326) (end 72.77256 69.95344) (width 0.254) (layer F.Cu) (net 7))
 (segment (start 72.77256 69.95344) (end 72.77256 71.906) (width 0.254) (layer F.Cu) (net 7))
 (segment (start 75.162 64.516) (end 75.162 67.564) (width 0.254) (layer B.Cu) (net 7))
 (segment (start 74.4 73.688) (end 74.4 68.326) (width 0.254) (layer B.Cu) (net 7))
 (segment (start 73.182 74.906) (end 74.4 73.688) (width 0.254) (layer B.Cu) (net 7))
 (segment (start 72.77256 74.906) (end 73.182 74.906) (width 0.254) (layer B.Cu) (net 7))
 (segment (start 71.352 69.85) (end 71.352 68.326) (width 0.254) (layer B.Cu) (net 5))
 (segment (start 71.352 68.326) (end 71.352 69.85) (width 0.254) (layer F.Cu) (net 5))
 (segment (start 71.27256 69.92944) (end 71.352 69.85) (width 0.254) (layer F.Cu) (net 5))
 (segment (start 71.27256 71.906) (end 71.27256 69.92944) (width 0.254) (layer F.Cu) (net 5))
 (segment (start 70.082 71.12) (end 71.352 69.85) (width 0.254) (layer B.Cu) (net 5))
 (segment (start 70.082 73.66) (end 70.082 71.12) (width 0.254) (layer B.Cu) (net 5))
 (segment (start 71.27256 74.85056) (end 70.082 73.66) (width 0.254) (layer B.Cu) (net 5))
 (segment (start 71.27256 74.906) (end 71.27256 74.85056) (width 0.254) (layer B.Cu) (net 5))
 (segment (start 71.098 66.802) (end 71.352 67.056) (width 0.254) (layer B.Cu) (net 5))
 (via (at 71.098 66.802) (size 0.889) (layers F.Cu B.Cu) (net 5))
 (segment (start 72.622 65.278) (end 71.098 66.802) (width 0.254) (layer F.Cu) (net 5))
 (segment (start 72.622 64.516) (end 72.622 65.278) (width 0.254) (layer F.Cu) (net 5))
 (segment (start 71.352 67.056) (end 71.098 66.802) (width 0.254) (layer F.Cu) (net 5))
 (segment (start 71.352 68.326) (end 71.352 67.056) (width 0.254) (layer F.Cu) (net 5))
 (segment (start 71.352 67.056) (end 71.098 66.802) (width 0.254) (layer B.Cu) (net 5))
 (segment (start 71.352 68.326) (end 71.352 67.056) (width 0.254) (layer B.Cu) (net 5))
 (segment (start 78.948 71.906) (end 80.07112 71.906) (width 0.254) (layer B.Cu) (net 10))
 (segment (start 78.718 72.136) (end 78.948 71.906) (width 0.254) (layer B.Cu) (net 10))
 (via (at 78.718 72.136) (size 0.889) (layers F.Cu B.Cu) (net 10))
 (segment (start 76.432 69.85) (end 78.718 72.136) (width 0.254) (layer F.Cu) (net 10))
 (segment (start 76.432 62.738) (end 76.432 69.85) (width 0.254) (layer F.Cu) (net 10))
 (segment (start 77.194 61.976) (end 76.432 62.738) (width 0.254) (layer F.Cu) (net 10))
 (segment (start 77.702 61.976) (end 77.194 61.976) (width 0.254) (layer F.Cu) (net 10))
 (segment (start 78.718 73.55288) (end 80.07112 74.906) (width 0.254) (layer F.Cu) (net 10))
 (segment (start 78.718 72.136) (end 78.718 73.55288) (width 0.254) (layer F.Cu) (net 10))
 (segment (start 81.766 67.818) (end 81.57112 68.01288) (width 0.254) (layer B.Cu) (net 12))
 (via (at 81.766 67.818) (size 0.889) (layers F.Cu B.Cu) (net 12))
 (segment (start 81.57112 68.01288) (end 81.57112 71.906) (width 0.254) (layer B.Cu) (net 12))
 (segment (start 81.258 67.31) (end 81.766 67.818) (width 0.254) (layer F.Cu) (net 12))
 (segment (start 80.242 67.31) (end 81.258 67.31) (width 0.254) (layer F.Cu) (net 12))
 (segment (start 78.972 66.04) (end 80.242 67.31) (width 0.254) (layer F.Cu) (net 12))
 (segment (start 78.972 63.246) (end 78.972 66.04) (width 0.254) (layer F.Cu) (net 12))
 (segment (start 80.242 61.976) (end 78.972 63.246) (width 0.254) (layer F.Cu) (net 12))
 (segment (start 81.57112 74.906) (end 82.044 74.906) (width 0.254) (layer F.Cu) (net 12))
 (segment (start 82.552 74.906) (end 83.798 73.66) (width 0.254) (layer F.Cu) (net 12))
 (segment (start 83.798 73.66) (end 83.798 68.834) (width 0.254) (layer F.Cu) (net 12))
 (segment (start 83.798 68.834) (end 82.782 67.818) (width 0.254) (layer F.Cu) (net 12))
 (segment (start 82.782 67.818) (end 81.766 67.818) (width 0.254) (layer F.Cu) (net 12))
 (segment (start 81.57112 74.906) (end 82.552 74.906) (width 0.254) (layer F.Cu) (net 12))
 (segment (start 80.242 65.786) (end 81.004 66.548) (width 0.254) (layer B.Cu) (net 11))
 (segment (start 81.004 66.548) (end 82.02 66.548) (width 0.254) (layer B.Cu) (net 11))
 (segment (start 82.02 66.548) (end 82.782 67.31) (width 0.254) (layer B.Cu) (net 11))
 (segment (start 82.782 67.31) (end 82.782 69.596) (width 0.254) (layer B.Cu) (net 11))
 (via (at 82.782 69.596) (size 0.889) (layers F.Cu B.Cu) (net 11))
 (segment (start 82.782 69.596) (end 81.57112 70.80688) (width 0.254) (layer F.Cu) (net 11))
 (segment (start 81.57112 70.80688) (end 81.57112 71.906) (width 0.254) (layer F.Cu) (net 11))
 (segment (start 80.242 64.516) (end 80.242 65.786) (width 0.254) (layer B.Cu) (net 11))
 (segment (start 82.782 73.69512) (end 81.57112 74.906) (width 0.254) (layer B.Cu) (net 11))
 (segment (start 82.782 69.596) (end 82.782 73.69512) (width 0.254) (layer B.Cu) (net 11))
 (segment (start 79.988 69.85) (end 79.988 68.326) (width 0.254) (layer B.Cu) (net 9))
 (segment (start 79.988 68.326) (end 79.988 69.85) (width 0.254) (layer F.Cu) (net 9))
 (segment (start 80.07112 69.93312) (end 79.988 69.85) (width 0.254) (layer F.Cu) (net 9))
 (segment (start 80.07112 71.906) (end 80.07112 69.93312) (width 0.254) (layer F.Cu) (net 9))
 (segment (start 78.972 69.85) (end 79.988 69.85) (width 0.254) (layer B.Cu) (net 9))
 (segment (start 77.702 71.12) (end 78.972 69.85) (width 0.254) (layer B.Cu) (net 9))
 (segment (start 77.702 72.644) (end 77.702 71.12) (width 0.254) (layer B.Cu) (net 9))
 (segment (start 79.964 74.906) (end 77.702 72.644) (width 0.254) (layer B.Cu) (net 9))
 (segment (start 80.07112 74.906) (end 79.964 74.906) (width 0.254) (layer B.Cu) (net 9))
 (segment (start 77.702 66.04) (end 79.988 68.326) (width 0.254) (layer B.Cu) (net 9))
 (segment (start 77.702 64.516) (end 77.702 66.04) (width 0.254) (layer B.Cu) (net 9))
 (segment (start 77.702 66.04) (end 79.988 68.326) (width 0.254) (layer F.Cu) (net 9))
 (segment (start 77.702 64.516) (end 77.702 66.04) (width 0.254) (layer F.Cu) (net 9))
 (segment (start 82.528 61.976) (end 82.782 61.976) (width 0.254) (layer F.Cu) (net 14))
 (segment (start 85.298 74.906) (end 84.56 74.168) (width 0.254) (layer F.Cu) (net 14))
 (segment (start 84.56 74.168) (end 84.56 67.564) (width 0.254) (layer F.Cu) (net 14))
 (segment (start 84.56 67.564) (end 82.782 65.786) (width 0.254) (layer F.Cu) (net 14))
 (segment (start 82.782 65.786) (end 81.512 65.786) (width 0.254) (layer F.Cu) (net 14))
 (segment (start 81.512 65.786) (end 81.512 64.77) (width 0.254) (layer F.Cu) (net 14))
 (segment (start 81.512 64.77) (end 81.512 62.992) (width 0.254) (layer F.Cu) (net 14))
 (segment (start 81.512 62.992) (end 82.528 61.976) (width 0.254) (layer F.Cu) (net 14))
 (segment (start 88.86968 74.906) (end 85.298 74.906) (width 0.254) (layer F.Cu) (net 14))
 (segment (start 82.528 61.976) (end 82.782 61.976) (width 0.254) (layer F.Cu) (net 14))
 (segment (start 81.512 62.992) (end 82.528 61.976) (width 0.254) (layer F.Cu) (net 14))
 (segment (start 81.512 65.786) (end 81.512 62.992) (width 0.254) (layer F.Cu) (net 14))
 (segment (start 82.782 65.786) (end 81.512 65.786) (width 0.254) (layer F.Cu) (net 14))
 (segment (start 84.56 67.564) (end 82.782 65.786) (width 0.254) (layer F.Cu) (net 14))
 (segment (start 87.124 71.906) (end 87.1 71.882) (width 0.254) (layer B.Cu) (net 14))
 (via (at 87.1 71.882) (size 0.889) (layers F.Cu B.Cu) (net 14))
 (segment (start 87.1 71.882) (end 84.56 71.882) (width 0.254) (layer F.Cu) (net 14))
 (segment (start 84.56 71.882) (end 84.56 67.564) (width 0.254) (layer F.Cu) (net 14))
 (segment (start 88.86968 71.906) (end 87.124 71.906) (width 0.254) (layer B.Cu) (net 14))
 (segment (start 90.36968 67.78568) (end 90.36968 71.906) (width 0.254) (layer B.Cu) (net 16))
 (segment (start 89.894 67.31) (end 90.36968 67.78568) (width 0.254) (layer B.Cu) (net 16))
 (segment (start 86.338 67.31) (end 89.894 67.31) (width 0.254) (layer B.Cu) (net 16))
 (segment (start 84.052 65.024) (end 86.338 67.31) (width 0.254) (layer B.Cu) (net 16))
 (segment (start 84.052 64.008) (end 84.052 65.024) (width 0.254) (layer B.Cu) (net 16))
 (segment (start 85.322 62.738) (end 84.052 64.008) (width 0.254) (layer B.Cu) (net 16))
 (segment (start 85.322 61.976) (end 85.322 62.738) (width 0.254) (layer B.Cu) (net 16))
 (segment (start 90.426 74.906) (end 90.36968 74.906) (width 0.254) (layer F.Cu) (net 16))
 (segment (start 86.338 62.992) (end 86.592 63.246) (width 0.254) (layer F.Cu) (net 16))
 (segment (start 86.592 63.246) (end 86.592 65.024) (width 0.254) (layer F.Cu) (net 16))
 (segment (start 86.592 65.024) (end 88.116 66.548) (width 0.254) (layer F.Cu) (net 16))
 (segment (start 88.116 66.548) (end 90.402 66.548) (width 0.254) (layer F.Cu) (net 16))
 (segment (start 90.402 66.548) (end 91.672 67.818) (width 0.254) (layer F.Cu) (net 16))
 (segment (start 91.672 67.818) (end 91.672 73.66) (width 0.254) (layer F.Cu) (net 16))
 (segment (start 91.672 73.66) (end 90.426 74.906) (width 0.254) (layer F.Cu) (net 16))
 (segment (start 85.322 61.976) (end 86.338 62.992) (width 0.254) (layer F.Cu) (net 16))
 (segment (start 90.36968 74.906) (end 90.426 74.906) (width 0.254) (layer B.Cu) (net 15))
 (segment (start 85.322 64.516) (end 85.322 64.77) (width 0.254) (layer B.Cu) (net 15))
 (segment (start 86.592 66.548) (end 90.402 66.548) (width 0.254) (layer B.Cu) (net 15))
 (segment (start 90.402 66.548) (end 91.672 67.818) (width 0.254) (layer B.Cu) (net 15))
 (segment (start 91.672 67.818) (end 91.672 73.60368) (width 0.254) (layer B.Cu) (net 15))
 (segment (start 91.672 73.60368) (end 90.36968 74.906) (width 0.254) (layer B.Cu) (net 15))
 (segment (start 85.322 65.278) (end 86.592 66.548) (width 0.254) (layer B.Cu) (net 15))
 (segment (start 85.322 64.516) (end 85.322 65.278) (width 0.254) (layer B.Cu) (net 15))
 (segment (start 85.343788 64.537788) (end 85.322 64.516) (width 0.254) (layer F.Cu) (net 15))
 (segment (start 90.36968 67.85032) (end 89.894 67.37464) (width 0.254) (layer F.Cu) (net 15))
 (segment (start 89.894 67.37464) (end 86.40264 67.37464) (width 0.254) (layer F.Cu) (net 15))
 (segment (start 86.40264 67.37464) (end 85.343788 66.315788) (width 0.254) (layer F.Cu) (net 15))
 (segment (start 85.343788 66.315788) (end 85.343788 64.537788) (width 0.254) (layer F.Cu) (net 15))
 (segment (start 90.36968 71.906) (end 90.36968 67.85032) (width 0.254) (layer F.Cu) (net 15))
 (segment (start 88.878 69.85) (end 88.878 68.326) (width 0.254) (layer B.Cu) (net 13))
 (segment (start 88.878 68.326) (end 88.878 69.85) (width 0.254) (layer F.Cu) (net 13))
 (segment (start 88.878 71.89768) (end 88.86968 71.906) (width 0.254) (layer F.Cu) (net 13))
 (segment (start 88.878 69.85) (end 88.878 71.89768) (width 0.254) (layer F.Cu) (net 13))
 (segment (start 88.86968 74.906) (end 88.6 74.906) (width 0.254) (layer B.Cu) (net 13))
 (segment (start 86.362 74.906) (end 86.084 74.628) (width 0.254) (layer B.Cu) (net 13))
 (segment (start 86.084 74.628) (end 86.084 70.612) (width 0.254) (layer B.Cu) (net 13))
 (segment (start 86.084 70.612) (end 86.846 69.85) (width 0.254) (layer B.Cu) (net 13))
 (segment (start 86.846 69.85) (end 88.878 69.85) (width 0.254) (layer B.Cu) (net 13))
 (segment (start 88.86968 74.906) (end 86.362 74.906) (width 0.254) (layer B.Cu) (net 13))
 (segment (start 85.576 68.326) (end 85.322 68.072) (width 0.254) (layer F.Cu) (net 13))
 (segment (start 85.322 68.072) (end 85.322 67.056) (width 0.254) (layer F.Cu) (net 13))
 (segment (start 85.322 67.056) (end 82.782 64.516) (width 0.254) (layer F.Cu) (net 13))
 (segment (start 88.878 68.326) (end 85.576 68.326) (width 0.254) (layer F.Cu) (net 13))
 (segment (start 82.782 64.516) (end 85.322 67.056) (width 0.254) (layer B.Cu) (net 13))
 (segment (start 85.576 68.326) (end 88.878 68.326) (width 0.254) (layer B.Cu) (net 13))
 (segment (start 85.322 68.072) (end 85.576 68.326) (width 0.254) (layer B.Cu) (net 13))
 (segment (start 85.322 67.056) (end 85.322 68.072) (width 0.254) (layer B.Cu) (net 13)))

